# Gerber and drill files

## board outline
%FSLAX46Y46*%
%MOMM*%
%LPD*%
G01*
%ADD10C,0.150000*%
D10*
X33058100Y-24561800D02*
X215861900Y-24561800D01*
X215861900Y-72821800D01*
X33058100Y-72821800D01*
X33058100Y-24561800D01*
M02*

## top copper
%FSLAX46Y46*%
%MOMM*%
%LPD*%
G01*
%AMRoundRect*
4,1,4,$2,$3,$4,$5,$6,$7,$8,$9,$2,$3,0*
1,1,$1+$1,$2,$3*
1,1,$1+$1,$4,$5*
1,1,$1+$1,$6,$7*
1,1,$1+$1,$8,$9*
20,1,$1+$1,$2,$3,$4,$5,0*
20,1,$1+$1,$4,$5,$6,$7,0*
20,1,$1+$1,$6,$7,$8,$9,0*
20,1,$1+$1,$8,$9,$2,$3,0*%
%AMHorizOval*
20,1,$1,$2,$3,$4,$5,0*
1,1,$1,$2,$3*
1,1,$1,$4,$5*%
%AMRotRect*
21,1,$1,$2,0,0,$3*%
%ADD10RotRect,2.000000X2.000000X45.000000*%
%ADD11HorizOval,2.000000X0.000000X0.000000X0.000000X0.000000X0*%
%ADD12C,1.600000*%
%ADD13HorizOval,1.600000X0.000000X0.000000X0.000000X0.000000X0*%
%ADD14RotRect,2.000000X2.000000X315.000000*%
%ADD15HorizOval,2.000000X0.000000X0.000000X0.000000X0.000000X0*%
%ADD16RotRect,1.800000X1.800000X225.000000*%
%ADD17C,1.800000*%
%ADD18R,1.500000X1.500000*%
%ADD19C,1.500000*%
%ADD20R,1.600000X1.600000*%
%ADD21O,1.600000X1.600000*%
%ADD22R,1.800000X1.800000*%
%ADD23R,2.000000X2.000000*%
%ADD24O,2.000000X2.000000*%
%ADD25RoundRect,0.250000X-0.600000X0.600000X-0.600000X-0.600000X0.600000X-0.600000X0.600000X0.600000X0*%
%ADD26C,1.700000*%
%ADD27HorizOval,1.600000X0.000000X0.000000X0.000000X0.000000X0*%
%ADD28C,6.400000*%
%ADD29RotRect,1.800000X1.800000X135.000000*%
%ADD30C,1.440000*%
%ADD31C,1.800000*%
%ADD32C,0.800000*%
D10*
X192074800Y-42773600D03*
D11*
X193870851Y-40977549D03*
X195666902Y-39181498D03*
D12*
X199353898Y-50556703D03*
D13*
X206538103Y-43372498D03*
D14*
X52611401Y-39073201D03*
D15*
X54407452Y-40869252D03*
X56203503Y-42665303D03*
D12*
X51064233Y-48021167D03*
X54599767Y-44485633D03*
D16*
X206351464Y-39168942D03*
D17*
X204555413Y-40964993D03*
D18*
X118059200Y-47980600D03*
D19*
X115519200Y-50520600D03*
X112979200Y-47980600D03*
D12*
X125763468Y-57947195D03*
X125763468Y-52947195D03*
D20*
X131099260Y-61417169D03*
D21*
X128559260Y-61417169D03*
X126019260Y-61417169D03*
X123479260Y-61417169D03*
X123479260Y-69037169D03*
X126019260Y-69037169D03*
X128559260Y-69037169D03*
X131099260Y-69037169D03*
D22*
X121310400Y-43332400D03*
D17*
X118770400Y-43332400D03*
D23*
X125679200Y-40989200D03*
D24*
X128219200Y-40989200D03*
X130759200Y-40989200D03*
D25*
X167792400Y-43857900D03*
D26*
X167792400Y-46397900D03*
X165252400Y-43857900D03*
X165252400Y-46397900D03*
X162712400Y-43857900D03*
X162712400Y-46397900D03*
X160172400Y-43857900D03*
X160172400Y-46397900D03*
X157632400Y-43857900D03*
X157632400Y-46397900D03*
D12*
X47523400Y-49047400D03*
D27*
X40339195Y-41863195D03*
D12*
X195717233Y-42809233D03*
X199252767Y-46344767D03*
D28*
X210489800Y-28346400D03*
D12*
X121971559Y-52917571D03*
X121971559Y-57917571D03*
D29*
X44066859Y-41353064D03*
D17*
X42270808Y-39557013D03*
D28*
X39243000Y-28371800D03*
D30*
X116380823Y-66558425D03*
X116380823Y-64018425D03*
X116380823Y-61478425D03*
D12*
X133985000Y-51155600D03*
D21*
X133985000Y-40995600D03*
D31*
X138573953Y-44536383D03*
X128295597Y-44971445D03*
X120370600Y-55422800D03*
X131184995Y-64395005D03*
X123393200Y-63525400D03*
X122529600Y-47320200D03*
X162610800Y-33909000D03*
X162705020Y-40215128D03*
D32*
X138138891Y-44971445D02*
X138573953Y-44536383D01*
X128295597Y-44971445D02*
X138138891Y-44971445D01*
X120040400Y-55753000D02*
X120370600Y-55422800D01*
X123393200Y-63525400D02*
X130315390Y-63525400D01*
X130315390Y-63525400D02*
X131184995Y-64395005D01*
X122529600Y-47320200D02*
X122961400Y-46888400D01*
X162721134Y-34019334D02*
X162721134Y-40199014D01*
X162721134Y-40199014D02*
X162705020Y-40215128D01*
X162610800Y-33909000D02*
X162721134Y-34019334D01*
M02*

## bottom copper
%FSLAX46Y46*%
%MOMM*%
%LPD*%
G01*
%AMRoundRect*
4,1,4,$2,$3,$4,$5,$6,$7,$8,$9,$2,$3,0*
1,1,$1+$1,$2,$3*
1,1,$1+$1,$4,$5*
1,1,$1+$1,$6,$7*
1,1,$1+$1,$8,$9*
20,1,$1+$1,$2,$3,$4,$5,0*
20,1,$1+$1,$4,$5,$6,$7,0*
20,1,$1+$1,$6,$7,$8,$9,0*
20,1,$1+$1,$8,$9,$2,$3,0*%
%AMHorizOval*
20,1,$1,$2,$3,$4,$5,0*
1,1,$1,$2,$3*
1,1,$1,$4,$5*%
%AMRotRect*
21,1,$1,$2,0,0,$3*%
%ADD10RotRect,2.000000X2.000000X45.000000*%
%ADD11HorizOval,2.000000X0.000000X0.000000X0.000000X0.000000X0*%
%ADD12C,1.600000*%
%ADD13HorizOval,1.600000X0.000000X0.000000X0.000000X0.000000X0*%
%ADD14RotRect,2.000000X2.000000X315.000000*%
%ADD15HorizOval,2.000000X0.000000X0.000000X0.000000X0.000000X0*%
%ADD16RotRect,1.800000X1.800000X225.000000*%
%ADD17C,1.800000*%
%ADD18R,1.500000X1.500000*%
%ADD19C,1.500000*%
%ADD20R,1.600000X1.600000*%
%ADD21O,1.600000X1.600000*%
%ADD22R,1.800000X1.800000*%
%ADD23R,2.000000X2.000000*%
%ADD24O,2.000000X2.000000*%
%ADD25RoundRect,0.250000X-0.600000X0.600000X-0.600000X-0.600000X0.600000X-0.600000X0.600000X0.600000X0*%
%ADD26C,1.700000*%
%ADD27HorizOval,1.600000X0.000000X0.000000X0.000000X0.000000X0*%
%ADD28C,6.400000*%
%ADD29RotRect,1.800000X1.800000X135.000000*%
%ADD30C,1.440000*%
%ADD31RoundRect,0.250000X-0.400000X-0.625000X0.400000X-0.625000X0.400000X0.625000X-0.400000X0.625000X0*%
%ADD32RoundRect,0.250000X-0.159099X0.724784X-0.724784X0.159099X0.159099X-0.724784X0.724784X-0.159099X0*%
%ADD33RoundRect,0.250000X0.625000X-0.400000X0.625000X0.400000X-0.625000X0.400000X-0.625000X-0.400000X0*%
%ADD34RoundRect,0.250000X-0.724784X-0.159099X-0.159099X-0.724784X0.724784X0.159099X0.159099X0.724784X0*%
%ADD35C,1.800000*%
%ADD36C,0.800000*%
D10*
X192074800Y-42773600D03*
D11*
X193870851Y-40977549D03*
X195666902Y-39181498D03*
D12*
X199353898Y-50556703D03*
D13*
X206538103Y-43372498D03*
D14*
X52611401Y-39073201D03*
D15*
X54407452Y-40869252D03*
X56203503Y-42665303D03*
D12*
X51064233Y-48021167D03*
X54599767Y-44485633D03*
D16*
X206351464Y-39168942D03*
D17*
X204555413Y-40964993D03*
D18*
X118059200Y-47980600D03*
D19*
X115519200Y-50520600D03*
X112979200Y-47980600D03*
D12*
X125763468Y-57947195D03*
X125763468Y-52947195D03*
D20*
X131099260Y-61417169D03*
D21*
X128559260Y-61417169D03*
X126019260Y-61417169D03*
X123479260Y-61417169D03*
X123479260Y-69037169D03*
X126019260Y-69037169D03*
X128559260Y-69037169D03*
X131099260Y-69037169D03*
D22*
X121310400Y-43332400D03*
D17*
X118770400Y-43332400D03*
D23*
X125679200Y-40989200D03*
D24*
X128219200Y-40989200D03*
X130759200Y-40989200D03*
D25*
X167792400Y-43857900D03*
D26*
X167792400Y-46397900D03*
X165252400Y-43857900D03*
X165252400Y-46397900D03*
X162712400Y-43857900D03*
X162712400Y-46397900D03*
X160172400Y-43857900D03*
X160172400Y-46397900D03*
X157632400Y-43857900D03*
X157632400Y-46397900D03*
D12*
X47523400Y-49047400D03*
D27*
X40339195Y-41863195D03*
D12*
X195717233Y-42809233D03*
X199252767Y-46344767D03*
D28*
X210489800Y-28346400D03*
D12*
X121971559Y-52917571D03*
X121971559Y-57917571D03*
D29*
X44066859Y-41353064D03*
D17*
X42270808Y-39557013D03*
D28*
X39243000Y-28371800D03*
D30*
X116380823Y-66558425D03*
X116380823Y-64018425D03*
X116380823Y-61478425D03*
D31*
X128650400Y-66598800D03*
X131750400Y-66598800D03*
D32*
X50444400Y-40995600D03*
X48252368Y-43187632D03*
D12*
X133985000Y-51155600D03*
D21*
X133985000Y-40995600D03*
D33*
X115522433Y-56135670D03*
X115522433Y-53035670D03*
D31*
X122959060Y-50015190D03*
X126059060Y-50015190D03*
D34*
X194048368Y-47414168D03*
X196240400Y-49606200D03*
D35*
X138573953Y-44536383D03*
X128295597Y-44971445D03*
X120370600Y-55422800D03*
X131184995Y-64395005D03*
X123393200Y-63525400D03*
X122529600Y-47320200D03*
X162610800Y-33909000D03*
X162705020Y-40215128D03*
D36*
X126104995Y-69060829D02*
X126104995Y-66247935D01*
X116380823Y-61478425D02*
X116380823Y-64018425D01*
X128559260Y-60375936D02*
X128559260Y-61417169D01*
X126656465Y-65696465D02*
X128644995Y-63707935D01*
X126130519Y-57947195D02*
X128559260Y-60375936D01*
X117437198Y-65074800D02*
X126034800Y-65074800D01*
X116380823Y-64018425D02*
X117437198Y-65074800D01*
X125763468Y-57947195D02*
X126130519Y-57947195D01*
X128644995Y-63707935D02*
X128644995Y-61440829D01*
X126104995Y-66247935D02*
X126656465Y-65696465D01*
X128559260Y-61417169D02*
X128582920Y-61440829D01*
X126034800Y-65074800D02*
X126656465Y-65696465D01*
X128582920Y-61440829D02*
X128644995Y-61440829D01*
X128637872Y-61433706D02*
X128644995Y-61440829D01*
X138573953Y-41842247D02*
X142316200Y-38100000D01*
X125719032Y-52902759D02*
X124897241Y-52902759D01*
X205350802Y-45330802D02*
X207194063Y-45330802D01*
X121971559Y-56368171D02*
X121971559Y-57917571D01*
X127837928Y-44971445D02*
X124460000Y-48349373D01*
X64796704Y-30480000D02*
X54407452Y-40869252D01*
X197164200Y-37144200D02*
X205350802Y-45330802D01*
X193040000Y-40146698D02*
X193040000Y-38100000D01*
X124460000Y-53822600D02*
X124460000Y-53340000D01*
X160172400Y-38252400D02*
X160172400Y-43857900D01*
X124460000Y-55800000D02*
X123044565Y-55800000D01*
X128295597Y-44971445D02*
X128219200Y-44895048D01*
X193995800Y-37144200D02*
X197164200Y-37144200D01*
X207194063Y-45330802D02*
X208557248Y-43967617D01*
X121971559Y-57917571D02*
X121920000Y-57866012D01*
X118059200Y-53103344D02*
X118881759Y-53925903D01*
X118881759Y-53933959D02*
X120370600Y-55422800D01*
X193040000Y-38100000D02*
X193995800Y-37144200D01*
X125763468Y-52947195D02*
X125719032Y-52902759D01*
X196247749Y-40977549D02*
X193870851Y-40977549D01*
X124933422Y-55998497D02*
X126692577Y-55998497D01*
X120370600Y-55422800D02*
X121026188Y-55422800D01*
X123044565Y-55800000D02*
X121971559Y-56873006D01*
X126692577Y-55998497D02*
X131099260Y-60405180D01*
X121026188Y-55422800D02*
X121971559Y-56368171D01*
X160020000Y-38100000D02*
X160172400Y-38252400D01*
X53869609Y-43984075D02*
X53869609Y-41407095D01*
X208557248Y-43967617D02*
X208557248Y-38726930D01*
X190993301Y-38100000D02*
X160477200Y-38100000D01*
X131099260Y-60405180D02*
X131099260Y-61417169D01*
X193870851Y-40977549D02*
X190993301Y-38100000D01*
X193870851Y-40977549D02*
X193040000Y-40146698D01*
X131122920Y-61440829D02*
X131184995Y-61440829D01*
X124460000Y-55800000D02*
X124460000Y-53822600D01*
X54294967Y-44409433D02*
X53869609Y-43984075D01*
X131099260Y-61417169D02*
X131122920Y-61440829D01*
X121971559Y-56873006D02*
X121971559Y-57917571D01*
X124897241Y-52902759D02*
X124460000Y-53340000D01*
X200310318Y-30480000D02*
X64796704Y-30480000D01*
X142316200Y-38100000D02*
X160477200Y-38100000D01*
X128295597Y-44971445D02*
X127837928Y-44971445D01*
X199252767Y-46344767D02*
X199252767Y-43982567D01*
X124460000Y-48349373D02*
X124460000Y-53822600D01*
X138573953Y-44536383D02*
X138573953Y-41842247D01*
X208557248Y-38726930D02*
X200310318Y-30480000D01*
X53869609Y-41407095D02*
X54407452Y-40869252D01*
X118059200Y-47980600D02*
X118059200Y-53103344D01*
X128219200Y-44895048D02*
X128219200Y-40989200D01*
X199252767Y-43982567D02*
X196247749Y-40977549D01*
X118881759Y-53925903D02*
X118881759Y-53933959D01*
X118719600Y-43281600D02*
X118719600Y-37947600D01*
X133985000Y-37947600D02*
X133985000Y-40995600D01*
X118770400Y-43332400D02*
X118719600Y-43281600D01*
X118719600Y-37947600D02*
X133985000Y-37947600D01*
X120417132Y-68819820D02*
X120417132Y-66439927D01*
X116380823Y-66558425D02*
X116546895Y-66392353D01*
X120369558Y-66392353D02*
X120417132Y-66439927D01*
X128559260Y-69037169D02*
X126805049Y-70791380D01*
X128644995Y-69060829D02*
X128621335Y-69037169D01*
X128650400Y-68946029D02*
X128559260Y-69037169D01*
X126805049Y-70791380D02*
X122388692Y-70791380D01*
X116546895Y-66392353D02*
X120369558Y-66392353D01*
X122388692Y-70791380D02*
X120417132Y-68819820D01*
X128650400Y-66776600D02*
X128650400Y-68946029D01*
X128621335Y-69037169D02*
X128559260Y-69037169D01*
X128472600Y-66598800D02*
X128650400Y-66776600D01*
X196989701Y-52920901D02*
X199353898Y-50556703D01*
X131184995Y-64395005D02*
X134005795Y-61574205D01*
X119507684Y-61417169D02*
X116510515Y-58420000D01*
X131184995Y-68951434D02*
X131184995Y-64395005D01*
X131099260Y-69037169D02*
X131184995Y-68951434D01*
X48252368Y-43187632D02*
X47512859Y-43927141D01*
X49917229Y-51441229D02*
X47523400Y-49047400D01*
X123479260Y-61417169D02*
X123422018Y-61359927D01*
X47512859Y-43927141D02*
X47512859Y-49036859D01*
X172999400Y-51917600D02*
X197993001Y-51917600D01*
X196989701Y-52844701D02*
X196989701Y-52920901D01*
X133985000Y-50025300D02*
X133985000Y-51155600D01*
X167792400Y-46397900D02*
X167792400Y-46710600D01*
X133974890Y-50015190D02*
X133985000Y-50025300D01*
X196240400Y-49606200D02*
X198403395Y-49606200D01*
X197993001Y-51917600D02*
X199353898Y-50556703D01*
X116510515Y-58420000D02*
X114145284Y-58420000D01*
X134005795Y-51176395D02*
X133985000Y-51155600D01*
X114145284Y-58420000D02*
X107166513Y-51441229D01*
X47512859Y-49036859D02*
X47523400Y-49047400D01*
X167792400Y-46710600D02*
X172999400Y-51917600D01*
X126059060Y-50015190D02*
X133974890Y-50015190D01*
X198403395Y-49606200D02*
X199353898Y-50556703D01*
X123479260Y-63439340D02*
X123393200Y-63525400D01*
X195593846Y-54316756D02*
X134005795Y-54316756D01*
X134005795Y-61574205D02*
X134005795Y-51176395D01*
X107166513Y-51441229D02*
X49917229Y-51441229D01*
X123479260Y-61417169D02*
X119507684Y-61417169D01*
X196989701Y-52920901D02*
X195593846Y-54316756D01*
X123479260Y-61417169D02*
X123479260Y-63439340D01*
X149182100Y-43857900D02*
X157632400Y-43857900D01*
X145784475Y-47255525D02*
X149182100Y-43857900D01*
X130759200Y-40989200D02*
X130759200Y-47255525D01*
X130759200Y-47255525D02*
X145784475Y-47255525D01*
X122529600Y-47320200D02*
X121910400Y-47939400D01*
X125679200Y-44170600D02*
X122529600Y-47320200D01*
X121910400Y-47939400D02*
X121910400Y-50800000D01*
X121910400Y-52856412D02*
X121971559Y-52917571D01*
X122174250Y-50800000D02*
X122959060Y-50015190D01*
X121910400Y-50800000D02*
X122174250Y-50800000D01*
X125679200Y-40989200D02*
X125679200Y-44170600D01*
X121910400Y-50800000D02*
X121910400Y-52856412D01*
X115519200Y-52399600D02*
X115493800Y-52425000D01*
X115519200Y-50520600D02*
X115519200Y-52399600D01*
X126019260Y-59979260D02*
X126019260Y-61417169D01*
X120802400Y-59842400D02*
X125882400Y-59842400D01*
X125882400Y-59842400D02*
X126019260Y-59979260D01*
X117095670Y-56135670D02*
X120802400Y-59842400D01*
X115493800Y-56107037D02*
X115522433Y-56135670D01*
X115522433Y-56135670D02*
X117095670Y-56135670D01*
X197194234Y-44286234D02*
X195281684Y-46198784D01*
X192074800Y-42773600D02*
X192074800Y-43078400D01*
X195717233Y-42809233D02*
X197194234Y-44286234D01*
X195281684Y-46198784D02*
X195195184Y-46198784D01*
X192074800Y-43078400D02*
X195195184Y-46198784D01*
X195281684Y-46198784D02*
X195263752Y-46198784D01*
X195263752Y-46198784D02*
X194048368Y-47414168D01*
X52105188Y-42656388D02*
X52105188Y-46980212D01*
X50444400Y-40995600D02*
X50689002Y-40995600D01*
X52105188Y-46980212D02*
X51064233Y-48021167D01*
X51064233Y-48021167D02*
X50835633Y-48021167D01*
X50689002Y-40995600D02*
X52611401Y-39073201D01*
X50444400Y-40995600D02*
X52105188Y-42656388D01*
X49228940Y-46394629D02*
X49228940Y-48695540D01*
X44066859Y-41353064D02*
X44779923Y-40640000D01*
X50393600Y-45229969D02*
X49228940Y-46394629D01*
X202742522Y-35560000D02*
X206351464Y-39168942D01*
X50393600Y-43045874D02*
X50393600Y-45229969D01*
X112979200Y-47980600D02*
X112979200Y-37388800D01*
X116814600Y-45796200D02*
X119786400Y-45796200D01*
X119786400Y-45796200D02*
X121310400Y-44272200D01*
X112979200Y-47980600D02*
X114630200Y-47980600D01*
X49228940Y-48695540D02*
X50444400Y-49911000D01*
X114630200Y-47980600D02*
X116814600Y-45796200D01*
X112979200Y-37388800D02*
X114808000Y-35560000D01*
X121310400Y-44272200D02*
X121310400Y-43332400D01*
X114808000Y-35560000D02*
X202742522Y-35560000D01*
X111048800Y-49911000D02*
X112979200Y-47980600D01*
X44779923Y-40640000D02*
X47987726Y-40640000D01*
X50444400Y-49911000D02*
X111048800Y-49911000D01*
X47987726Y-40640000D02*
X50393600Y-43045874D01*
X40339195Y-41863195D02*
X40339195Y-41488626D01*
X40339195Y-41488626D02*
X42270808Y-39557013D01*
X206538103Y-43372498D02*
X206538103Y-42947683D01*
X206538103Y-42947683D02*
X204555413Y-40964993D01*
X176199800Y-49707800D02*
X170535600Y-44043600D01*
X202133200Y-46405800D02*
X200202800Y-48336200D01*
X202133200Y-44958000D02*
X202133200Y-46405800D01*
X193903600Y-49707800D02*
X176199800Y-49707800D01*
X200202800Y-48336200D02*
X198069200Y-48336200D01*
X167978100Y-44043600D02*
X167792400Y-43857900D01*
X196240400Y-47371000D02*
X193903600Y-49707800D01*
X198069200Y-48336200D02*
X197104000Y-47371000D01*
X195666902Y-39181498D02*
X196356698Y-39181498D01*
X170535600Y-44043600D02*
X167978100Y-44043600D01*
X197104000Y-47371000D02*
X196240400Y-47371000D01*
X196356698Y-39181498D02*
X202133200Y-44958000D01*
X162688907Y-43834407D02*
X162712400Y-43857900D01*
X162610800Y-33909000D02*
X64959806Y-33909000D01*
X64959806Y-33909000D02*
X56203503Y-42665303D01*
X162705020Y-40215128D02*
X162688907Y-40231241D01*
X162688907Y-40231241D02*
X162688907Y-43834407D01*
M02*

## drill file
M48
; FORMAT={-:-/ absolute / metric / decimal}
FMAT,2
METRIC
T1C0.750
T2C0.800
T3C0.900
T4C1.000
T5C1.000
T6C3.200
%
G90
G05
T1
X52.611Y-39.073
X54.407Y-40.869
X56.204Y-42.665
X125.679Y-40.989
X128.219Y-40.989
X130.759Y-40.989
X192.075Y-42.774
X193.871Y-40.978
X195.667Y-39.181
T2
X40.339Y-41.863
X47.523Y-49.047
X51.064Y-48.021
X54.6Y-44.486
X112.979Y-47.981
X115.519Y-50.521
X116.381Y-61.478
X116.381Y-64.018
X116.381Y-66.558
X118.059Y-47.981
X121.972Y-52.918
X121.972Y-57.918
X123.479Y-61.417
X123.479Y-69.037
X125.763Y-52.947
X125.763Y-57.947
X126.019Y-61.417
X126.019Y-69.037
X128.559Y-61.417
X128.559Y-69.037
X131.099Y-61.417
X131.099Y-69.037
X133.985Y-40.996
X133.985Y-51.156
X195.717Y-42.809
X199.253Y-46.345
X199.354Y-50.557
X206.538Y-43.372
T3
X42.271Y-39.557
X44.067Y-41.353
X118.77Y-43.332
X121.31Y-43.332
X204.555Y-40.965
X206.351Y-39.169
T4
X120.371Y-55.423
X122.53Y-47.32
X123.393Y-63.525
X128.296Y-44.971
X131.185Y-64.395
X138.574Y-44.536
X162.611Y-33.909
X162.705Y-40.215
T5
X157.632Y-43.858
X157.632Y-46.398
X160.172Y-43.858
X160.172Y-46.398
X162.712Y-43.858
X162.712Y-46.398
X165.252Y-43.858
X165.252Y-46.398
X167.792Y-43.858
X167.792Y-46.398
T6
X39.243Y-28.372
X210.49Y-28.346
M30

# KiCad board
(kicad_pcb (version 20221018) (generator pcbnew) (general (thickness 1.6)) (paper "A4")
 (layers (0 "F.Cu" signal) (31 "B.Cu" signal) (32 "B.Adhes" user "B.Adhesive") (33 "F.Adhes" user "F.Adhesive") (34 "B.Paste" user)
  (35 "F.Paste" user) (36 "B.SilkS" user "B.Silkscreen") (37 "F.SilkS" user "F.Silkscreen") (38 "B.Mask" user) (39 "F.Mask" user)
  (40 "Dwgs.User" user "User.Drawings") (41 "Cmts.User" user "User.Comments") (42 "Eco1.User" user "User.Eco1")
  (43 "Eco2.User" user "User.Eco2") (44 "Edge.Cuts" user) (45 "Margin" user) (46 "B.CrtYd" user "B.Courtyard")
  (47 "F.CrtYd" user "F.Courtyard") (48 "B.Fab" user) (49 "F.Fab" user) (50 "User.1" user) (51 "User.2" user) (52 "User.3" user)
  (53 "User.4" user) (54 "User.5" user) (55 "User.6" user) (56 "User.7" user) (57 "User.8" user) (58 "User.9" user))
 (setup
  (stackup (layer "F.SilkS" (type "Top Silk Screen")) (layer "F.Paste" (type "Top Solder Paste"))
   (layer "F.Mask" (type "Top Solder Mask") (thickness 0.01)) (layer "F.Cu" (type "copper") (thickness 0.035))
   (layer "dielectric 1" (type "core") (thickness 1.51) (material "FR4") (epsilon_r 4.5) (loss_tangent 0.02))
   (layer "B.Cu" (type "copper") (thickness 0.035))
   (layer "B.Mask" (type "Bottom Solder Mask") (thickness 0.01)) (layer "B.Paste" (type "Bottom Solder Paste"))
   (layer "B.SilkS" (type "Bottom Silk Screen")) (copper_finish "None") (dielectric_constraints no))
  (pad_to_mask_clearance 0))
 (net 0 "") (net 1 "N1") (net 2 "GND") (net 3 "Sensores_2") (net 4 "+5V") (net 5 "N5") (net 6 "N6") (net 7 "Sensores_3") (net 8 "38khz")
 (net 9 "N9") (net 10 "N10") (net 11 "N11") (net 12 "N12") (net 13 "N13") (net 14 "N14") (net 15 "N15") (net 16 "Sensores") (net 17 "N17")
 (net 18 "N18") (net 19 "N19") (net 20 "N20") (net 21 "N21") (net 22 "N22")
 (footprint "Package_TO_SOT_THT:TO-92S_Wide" (layer "F.Cu") (at 192.0748 42.7736 45)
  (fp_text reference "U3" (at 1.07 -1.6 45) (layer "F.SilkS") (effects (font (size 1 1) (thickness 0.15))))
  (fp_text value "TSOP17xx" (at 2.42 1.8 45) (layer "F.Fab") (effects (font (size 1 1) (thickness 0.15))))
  (pad "1" thru_hole rect (at 0 0 45) (size 2 2) (drill 0.75) (layers "*.Cu" "*.Mask") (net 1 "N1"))
  (pad "2" thru_hole oval (at 2.54 0 45) (size 2 2) (drill 0.75) (layers "*.Cu" "*.Mask") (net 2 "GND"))
  (pad "3" thru_hole oval (at 5.079999 0 45) (size 2 2) (drill 0.75) (layers "*.Cu" "*.Mask") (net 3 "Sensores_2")))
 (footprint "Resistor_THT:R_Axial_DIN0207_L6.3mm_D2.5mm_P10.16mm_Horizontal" (layer "F.Cu") (at 199.353898 50.556703 45)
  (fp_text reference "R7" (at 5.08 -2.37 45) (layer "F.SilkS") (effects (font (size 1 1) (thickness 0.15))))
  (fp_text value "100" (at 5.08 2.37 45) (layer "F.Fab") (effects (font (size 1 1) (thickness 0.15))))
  (pad "1" thru_hole circle (at 0 0 45) (size 1.6 1.6) (drill 0.8) (layers "*.Cu" "*.Mask") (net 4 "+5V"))
  (pad "2" thru_hole oval (at 10.16 0 45) (size 1.6 1.6) (drill 0.8) (layers "*.Cu" "*.Mask") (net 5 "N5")))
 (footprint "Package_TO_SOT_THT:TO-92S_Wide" (layer "F.Cu") (at 52.611401 39.073201 -45)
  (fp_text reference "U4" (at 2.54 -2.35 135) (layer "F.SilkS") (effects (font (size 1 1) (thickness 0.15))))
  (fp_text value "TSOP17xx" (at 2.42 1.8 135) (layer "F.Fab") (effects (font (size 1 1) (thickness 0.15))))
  (pad "1" thru_hole rect (at 0 0 315) (size 2 2) (drill 0.75) (layers "*.Cu" "*.Mask") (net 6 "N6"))
  (pad "2" thru_hole oval (at 2.54 0 315) (size 2 2) (drill 0.75) (layers "*.Cu" "*.Mask") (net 2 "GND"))
  (pad "3" thru_hole oval (at 5.079999 0 315) (size 2 2) (drill 0.75) (layers "*.Cu" "*.Mask") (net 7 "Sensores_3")))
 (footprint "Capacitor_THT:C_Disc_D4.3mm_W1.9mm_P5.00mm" (layer "F.Cu") (at 51.064233 48.021167 45)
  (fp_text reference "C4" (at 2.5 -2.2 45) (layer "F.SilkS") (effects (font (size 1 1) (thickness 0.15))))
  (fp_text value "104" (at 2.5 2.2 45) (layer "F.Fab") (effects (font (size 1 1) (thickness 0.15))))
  (pad "1" thru_hole circle (at 0 0 45) (size 1.6 1.6) (drill 0.8) (layers "*.Cu" "*.Mask") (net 6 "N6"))
  (pad "2" thru_hole circle (at 5 0 45) (size 1.6 1.6) (drill 0.8) (layers "*.Cu" "*.Mask") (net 2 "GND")))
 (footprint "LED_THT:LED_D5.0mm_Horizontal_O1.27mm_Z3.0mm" (layer "F.Cu") (at 206.351464 39.168942 -135)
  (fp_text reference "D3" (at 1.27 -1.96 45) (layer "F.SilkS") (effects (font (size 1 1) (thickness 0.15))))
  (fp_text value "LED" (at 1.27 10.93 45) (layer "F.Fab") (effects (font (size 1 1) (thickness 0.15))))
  (pad "1" thru_hole rect (at 0 0 225) (size 1.8 1.8) (drill 0.9) (layers "*.Cu" "*.Mask") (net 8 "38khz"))
  (pad "2" thru_hole circle (at 2.54 0 225) (size 1.8 1.8) (drill 0.9) (layers "*.Cu" "*.Mask") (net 5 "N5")))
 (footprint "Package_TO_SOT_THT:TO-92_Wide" (layer "F.Cu") (at 118.0592 47.9806 180)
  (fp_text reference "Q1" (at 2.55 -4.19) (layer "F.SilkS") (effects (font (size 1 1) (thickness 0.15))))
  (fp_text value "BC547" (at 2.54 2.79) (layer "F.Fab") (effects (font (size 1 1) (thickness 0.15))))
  (pad "1" thru_hole rect (at 0 0 180) (size 1.5 1.5) (drill 0.8) (layers "*.Cu" "*.Mask") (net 2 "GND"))
  (pad "2" thru_hole circle (at 2.54 -2.54 180) (size 1.5 1.5) (drill 0.8) (layers "*.Cu" "*.Mask") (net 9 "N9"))
  (pad "3" thru_hole circle (at 5.08 0 180) (size 1.5 1.5) (drill 0.8) (layers "*.Cu" "*.Mask") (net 8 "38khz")))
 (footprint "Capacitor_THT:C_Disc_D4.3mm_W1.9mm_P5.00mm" (layer "F.Cu") (at 125.763468 57.947195 90)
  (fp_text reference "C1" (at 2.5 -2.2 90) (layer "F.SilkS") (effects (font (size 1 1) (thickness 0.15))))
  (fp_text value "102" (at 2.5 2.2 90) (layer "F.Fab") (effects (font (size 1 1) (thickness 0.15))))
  (pad "1" thru_hole circle (at 0 0 90) (size 1.6 1.6) (drill 0.8) (layers "*.Cu" "*.Mask") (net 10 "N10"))
  (pad "2" thru_hole circle (at 5 0 90) (size 1.6 1.6) (drill 0.8) (layers "*.Cu" "*.Mask") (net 2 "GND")))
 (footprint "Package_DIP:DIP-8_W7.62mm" (layer "F.Cu") (at 131.09926 61.417169 -90)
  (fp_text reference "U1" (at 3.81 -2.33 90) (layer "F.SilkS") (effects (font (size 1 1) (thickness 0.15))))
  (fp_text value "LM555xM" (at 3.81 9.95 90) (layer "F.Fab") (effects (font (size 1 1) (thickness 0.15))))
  (pad "1" thru_hole rect (at 0 0 270) (size 1.6 1.6) (drill 0.8) (layers "*.Cu" "*.Mask") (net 2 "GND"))
  (pad "2" thru_hole oval (at 0 2.54 270) (size 1.6 1.6) (drill 0.8) (layers "*.Cu" "*.Mask") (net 10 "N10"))
  (pad "3" thru_hole oval (at 0 5.08 270) (size 1.6 1.6) (drill 0.8) (layers "*.Cu" "*.Mask") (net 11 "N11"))
  (pad "4" thru_hole oval (at 0 7.62 270) (size 1.6 1.6) (drill 0.8) (layers "*.Cu" "*.Mask") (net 4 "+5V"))
  (pad "5" thru_hole oval (at 7.62 7.62 270) (size 1.6 1.6) (drill 0.8) (layers "*.Cu" "*.Mask") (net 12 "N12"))
  (pad "6" thru_hole oval (at 7.62 5.08 270) (size 1.6 1.6) (drill 0.8) (layers "*.Cu" "*.Mask") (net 10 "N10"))
  (pad "7" thru_hole oval (at 7.62 2.54 270) (size 1.6 1.6) (drill 0.8) (layers "*.Cu" "*.Mask") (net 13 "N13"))
  (pad "8" thru_hole oval (at 7.62 0 270) (size 1.6 1.6) (drill 0.8) (layers "*.Cu" "*.Mask") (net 4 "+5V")))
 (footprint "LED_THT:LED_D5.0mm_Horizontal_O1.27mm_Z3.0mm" (layer "F.Cu") (at 121.3104 43.3324 180)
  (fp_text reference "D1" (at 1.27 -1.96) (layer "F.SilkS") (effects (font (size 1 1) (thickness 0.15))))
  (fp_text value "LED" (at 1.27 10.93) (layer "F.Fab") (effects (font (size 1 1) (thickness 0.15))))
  (pad "1" thru_hole rect (at 0 0 180) (size 1.8 1.8) (drill 0.9) (layers "*.Cu" "*.Mask") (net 8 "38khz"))
  (pad "2" thru_hole circle (at 2.54 0 180) (size 1.8 1.8) (drill 0.9) (layers "*.Cu" "*.Mask") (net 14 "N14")))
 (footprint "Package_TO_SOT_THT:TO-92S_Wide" (layer "F.Cu") (at 125.6792 40.9892)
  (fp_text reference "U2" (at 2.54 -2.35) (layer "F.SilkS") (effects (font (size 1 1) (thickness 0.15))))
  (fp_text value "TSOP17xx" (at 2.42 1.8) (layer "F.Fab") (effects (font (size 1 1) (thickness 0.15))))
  (pad "1" thru_hole rect (at 0 0) (size 2 2) (drill 0.75) (layers "*.Cu" "*.Mask") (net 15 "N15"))
  (pad "2" thru_hole oval (at 2.54 0) (size 2 2) (drill 0.75) (layers "*.Cu" "*.Mask") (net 2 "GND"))
  (pad "3" thru_hole oval (at 5.08 0) (size 2 2) (drill 0.75) (layers "*.Cu" "*.Mask") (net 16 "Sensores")))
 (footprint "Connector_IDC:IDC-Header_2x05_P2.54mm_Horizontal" (layer "F.Cu") (at 167.7924 43.8579 -90)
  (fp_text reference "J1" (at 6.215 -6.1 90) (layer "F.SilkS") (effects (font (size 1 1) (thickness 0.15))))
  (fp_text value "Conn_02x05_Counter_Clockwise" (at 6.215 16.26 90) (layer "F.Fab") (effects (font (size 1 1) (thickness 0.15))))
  (pad "1" thru_hole roundrect (at 0 0 270) (size 1.7 1.7) (drill 1) (layers "*.Cu" "*.Mask") (roundrect_rratio 0.147059)
   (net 3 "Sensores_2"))
  (pad "2" thru_hole circle (at 2.54 0 270) (size 1.7 1.7) (drill 1) (layers "*.Cu" "*.Mask") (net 4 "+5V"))
  (pad "3" thru_hole circle (at 0 2.54 270) (size 1.7 1.7) (drill 1) (layers "*.Cu" "*.Mask") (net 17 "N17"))
  (pad "4" thru_hole circle (at 2.54 2.54 270) (size 1.7 1.7) (drill 1) (layers "*.Cu" "*.Mask") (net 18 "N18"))
  (pad "5" thru_hole circle (at 0 5.08 270) (size 1.7 1.7) (drill 1) (layers "*.Cu" "*.Mask") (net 7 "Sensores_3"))
  (pad "6" thru_hole circle (at 2.54 5.08 270) (size 1.7 1.7) (drill 1) (layers "*.Cu" "*.Mask") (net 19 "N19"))
  (pad "7" thru_hole circle (at 0 7.62 270) (size 1.7 1.7) (drill 1) (layers "*.Cu" "*.Mask") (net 2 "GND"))
  (pad "8" thru_hole circle (at 2.54 7.62 270) (size 1.7 1.7) (drill 1) (layers "*.Cu" "*.Mask") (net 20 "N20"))
  (pad "9" thru_hole circle (at 0 10.16 270) (size 1.7 1.7) (drill 1) (layers "*.Cu" "*.Mask") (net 16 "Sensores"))
  (pad "10" thru_hole circle (at 2.54 10.16 270) (size 1.7 1.7) (drill 1) (layers "*.Cu" "*.Mask") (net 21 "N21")))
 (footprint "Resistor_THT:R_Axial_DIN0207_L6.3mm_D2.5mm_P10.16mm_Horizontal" (layer "F.Cu") (at 47.5234 49.0474 135)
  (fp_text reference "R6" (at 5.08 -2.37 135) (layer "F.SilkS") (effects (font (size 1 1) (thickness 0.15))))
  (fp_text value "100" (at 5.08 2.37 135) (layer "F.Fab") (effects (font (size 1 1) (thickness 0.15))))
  (pad "1" thru_hole circle (at 0 0 135) (size 1.6 1.6) (drill 0.8) (layers "*.Cu" "*.Mask") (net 4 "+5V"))
  (pad "2" thru_hole oval (at 10.16 0 135) (size 1.6 1.6) (drill 0.8) (layers "*.Cu" "*.Mask") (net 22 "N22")))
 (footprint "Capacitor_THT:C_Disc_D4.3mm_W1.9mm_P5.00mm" (layer "F.Cu") (at 195.717233 42.809233 -45)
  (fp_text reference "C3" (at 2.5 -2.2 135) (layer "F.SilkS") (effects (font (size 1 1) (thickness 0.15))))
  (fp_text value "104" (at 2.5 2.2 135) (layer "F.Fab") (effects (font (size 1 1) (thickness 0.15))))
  (pad "1" thru_hole circle (at 0 0 315) (size 1.6 1.6) (drill 0.8) (layers "*.Cu" "*.Mask") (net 1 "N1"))
  (pad "2" thru_hole circle (at 5 0 315) (size 1.6 1.6) (drill 0.8) (layers "*.Cu" "*.Mask") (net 2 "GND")))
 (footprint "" (layer "F.Cu") (at 210.4898 28.3464 180)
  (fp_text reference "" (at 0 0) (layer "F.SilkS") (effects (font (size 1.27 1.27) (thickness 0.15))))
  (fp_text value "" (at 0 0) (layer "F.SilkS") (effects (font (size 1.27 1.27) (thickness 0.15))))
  (pad "1" thru_hole circle (at 0 0 180) (size 6.4 6.4) (drill 3.2) (layers "*.Cu" "*.Mask")))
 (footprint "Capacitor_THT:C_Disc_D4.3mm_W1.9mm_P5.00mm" (layer "F.Cu") (at 121.971559 52.917571 -90)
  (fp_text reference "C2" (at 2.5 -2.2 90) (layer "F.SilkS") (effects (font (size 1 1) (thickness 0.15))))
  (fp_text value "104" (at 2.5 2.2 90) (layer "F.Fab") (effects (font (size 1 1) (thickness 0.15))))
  (pad "1" thru_hole circle (at 0 0 270) (size 1.6 1.6) (drill 0.8) (layers "*.Cu" "*.Mask") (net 15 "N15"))
  (pad "2" thru_hole circle (at 5 0 270) (size 1.6 1.6) (drill 0.8) (layers "*.Cu" "*.Mask") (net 2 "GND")))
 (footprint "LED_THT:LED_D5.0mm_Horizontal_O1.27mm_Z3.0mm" (layer "F.Cu") (at 44.066859 41.353064 135)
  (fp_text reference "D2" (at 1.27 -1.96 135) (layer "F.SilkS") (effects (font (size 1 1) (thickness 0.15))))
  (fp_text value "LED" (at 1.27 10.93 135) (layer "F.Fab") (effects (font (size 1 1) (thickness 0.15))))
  (pad "1" thru_hole rect (at 0 0 135) (size 1.8 1.8) (drill 0.9) (layers "*.Cu" "*.Mask") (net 8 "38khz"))
  (pad "2" thru_hole circle (at 2.54 0 135) (size 1.8 1.8) (drill 0.9) (layers "*.Cu" "*.Mask") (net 22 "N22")))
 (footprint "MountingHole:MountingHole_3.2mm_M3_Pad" (layer "F.Cu") (at 39.243 28.3718 180)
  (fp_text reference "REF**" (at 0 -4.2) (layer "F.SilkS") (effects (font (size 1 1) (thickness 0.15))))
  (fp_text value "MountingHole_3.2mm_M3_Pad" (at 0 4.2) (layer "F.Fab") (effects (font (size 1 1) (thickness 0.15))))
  (pad "1" thru_hole circle (at 0 0 180) (size 6.4 6.4) (drill 3.2) (layers "*.Cu" "*.Mask")))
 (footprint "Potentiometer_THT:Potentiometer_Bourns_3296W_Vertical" (layer "F.Cu") (at 116.380823 66.558425 -90)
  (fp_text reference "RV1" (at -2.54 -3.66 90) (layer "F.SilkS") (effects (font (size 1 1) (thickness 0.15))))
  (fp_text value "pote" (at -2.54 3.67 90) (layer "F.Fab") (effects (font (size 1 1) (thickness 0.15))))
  (pad "1" thru_hole circle (at 0 0 270) (size 1.44 1.44) (drill 0.8) (layers "*.Cu" "*.Mask") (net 13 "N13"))
  (pad "2" thru_hole circle (at -2.54 0 270) (size 1.44 1.44) (drill 0.8) (layers "*.Cu" "*.Mask") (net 10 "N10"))
  (pad "3" thru_hole circle (at -5.08 0 270) (size 1.44 1.44) (drill 0.8) (layers "*.Cu" "*.Mask") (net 10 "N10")))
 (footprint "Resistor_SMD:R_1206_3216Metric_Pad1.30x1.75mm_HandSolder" (layer "B.Cu") (at 130.2004 66.5988)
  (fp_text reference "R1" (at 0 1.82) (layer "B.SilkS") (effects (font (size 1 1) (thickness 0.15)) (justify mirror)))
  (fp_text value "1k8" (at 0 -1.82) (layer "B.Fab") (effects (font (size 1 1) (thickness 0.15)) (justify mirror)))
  (pad "1" smd roundrect (at -1.55 0) (size 1.3 1.75) (layers "B.Cu" "B.Paste" "B.Mask") (roundrect_rratio 0.192308) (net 13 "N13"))
  (pad "2" smd roundrect (at 1.55 0) (size 1.3 1.75) (layers "B.Cu" "B.Paste" "B.Mask") (roundrect_rratio 0.192308) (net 4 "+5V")))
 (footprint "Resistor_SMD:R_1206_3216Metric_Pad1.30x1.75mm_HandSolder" (layer "B.Cu") (at 49.348384 42.091616 -135)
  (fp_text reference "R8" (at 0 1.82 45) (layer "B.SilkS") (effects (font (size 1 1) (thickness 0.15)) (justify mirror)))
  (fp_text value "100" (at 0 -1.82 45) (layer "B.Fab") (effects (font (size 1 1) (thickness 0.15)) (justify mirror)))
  (pad "1" smd roundrect (at -1.55 0 225) (size 1.3 1.75) (layers "B.Cu" "B.Paste" "B.Mask") (roundrect_rratio 0.192308) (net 6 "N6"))
  (pad "2" smd roundrect (at 1.55 0 225) (size 1.3 1.75) (layers "B.Cu" "B.Paste" "B.Mask") (roundrect_rratio 0.192308) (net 4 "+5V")))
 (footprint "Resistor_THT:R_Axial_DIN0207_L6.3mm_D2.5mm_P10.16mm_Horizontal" (layer "B.Cu") (at 133.985 51.1556 90)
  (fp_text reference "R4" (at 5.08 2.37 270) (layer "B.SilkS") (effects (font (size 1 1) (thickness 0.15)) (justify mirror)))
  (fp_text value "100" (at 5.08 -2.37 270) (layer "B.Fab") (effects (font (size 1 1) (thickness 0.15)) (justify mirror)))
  (pad "1" thru_hole circle (at 0 0 90) (size 1.6 1.6) (drill 0.8) (layers "*.Cu" "*.Mask") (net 4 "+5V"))
  (pad "2" thru_hole oval (at 10.16 0 90) (size 1.6 1.6) (drill 0.8) (layers "*.Cu" "*.Mask") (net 14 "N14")))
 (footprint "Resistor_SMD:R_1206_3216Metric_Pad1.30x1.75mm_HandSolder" (layer "B.Cu") (at 115.522433 54.58567 90)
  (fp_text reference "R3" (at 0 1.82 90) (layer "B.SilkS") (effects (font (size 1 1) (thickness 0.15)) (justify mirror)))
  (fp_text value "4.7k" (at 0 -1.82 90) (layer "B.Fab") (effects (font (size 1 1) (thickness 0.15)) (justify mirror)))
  (pad "1" smd roundrect (at -1.55 0 90) (size 1.3 1.75) (layers "B.Cu" "B.Paste" "B.Mask") (roundrect_rratio 0.192308) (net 11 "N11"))
  (pad "2" smd roundrect (at 1.55 0 90) (size 1.3 1.75) (layers "B.Cu" "B.Paste" "B.Mask") (roundrect_rratio 0.192308) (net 9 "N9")))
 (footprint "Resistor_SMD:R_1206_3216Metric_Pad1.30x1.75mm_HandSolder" (layer "B.Cu") (at 124.50906 50.01519)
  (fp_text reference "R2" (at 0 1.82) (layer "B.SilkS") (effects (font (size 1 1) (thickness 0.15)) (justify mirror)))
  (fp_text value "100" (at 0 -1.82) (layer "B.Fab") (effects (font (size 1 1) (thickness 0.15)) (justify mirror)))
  (pad "1" smd roundrect (at -1.55 0) (size 1.3 1.75) (layers "B.Cu" "B.Paste" "B.Mask") (roundrect_rratio 0.192308) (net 15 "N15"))
  (pad "2" smd roundrect (at 1.55 0) (size 1.3 1.75) (layers "B.Cu" "B.Paste" "B.Mask") (roundrect_rratio 0.192308) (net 4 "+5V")))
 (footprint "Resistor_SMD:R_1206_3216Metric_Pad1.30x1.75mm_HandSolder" (layer "B.Cu") (at 195.144384 48.510184 -45)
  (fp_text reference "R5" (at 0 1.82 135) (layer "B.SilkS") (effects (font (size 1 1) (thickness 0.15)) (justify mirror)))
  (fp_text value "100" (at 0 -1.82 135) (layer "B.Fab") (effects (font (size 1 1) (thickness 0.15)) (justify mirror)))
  (pad "1" smd roundrect (at -1.55 0 315) (size 1.3 1.75) (layers "B.Cu" "B.Paste" "B.Mask") (roundrect_rratio 0.192308) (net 1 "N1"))
  (pad "2" smd roundrect (at 1.55 0 315) (size 1.3 1.75) (layers "B.Cu" "B.Paste" "B.Mask") (roundrect_rratio 0.192308) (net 4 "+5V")))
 (gr_rect (start 33.0581 24.5618) (end 215.8619 72.8218) (stroke (width 0.15) (type default)) (fill none) (layer "Edge.Cuts"))
 (segment (start 126.104995 69.060829) (end 126.104995 66.247935) (width 0.8) (layer "B.Cu") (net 10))
 (segment (start 116.380823 61.478425) (end 116.380823 64.018425) (width 0.8) (layer "B.Cu") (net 10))
 (segment (start 128.55926 60.375936) (end 128.55926 61.417169) (width 0.8) (layer "B.Cu") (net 10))
 (segment (start 126.656465 65.696465) (end 128.644995 63.707935) (width 0.8) (layer "B.Cu") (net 10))
 (segment (start 126.130519 57.947195) (end 128.55926 60.375936) (width 0.8) (layer "B.Cu") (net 10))
 (segment (start 117.437198 65.0748) (end 126.0348 65.0748) (width 0.8) (layer "B.Cu") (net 10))
 (segment (start 116.380823 64.018425) (end 117.437198 65.0748) (width 0.8) (layer "B.Cu") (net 10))
 (segment (start 125.763468 57.947195) (end 126.130519 57.947195) (width 0.8) (layer "B.Cu") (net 10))
 (segment (start 128.644995 63.707935) (end 128.644995 61.440829) (width 0.8) (layer "B.Cu") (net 10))
 (segment (start 126.104995 66.247935) (end 126.656465 65.696465) (width 0.8) (layer "B.Cu") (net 10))
 (segment (start 128.55926 61.417169) (end 128.58292 61.440829) (width 0.8) (layer "B.Cu") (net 10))
 (segment (start 126.0348 65.0748) (end 126.656465 65.696465) (width 0.8) (layer "B.Cu") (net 10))
 (segment (start 128.58292 61.440829) (end 128.644995 61.440829) (width 0.8) (layer "B.Cu") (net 10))
 (segment (start 128.637872 61.433706) (end 128.644995 61.440829) (width 0.8) (layer "B.Cu") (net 10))
 (segment (start 138.138891 44.971445) (end 138.573953 44.536383) (width 0.8) (layer "F.Cu") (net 2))
 (segment (start 128.295597 44.971445) (end 138.138891 44.971445) (width 0.8) (layer "F.Cu") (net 2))
 (segment (start 120.0404 55.753) (end 120.3706 55.4228) (width 0.8) (layer "F.Cu") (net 2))
 (via (at 138.573953 44.536383) (size 1.8) (drill 1) (layers "F.Cu" "B.Cu") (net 2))
 (via (at 128.295597 44.971445) (size 1.8) (drill 1) (layers "F.Cu" "B.Cu") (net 2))
 (via (at 120.3706 55.4228) (size 1.8) (drill 1) (layers "F.Cu" "B.Cu") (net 2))
 (segment (start 138.573953 41.842247) (end 142.3162 38.1) (width 0.8) (layer "B.Cu") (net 2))
 (segment (start 125.719032 52.902759) (end 124.897241 52.902759) (width 0.8) (layer "B.Cu") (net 2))
 (segment (start 205.350802 45.330802) (end 207.194063 45.330802) (width 0.8) (layer "B.Cu") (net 2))
 (segment (start 121.971559 56.368171) (end 121.971559 57.917571) (width 0.8) (layer "B.Cu") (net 2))
 (segment (start 127.837928 44.971445) (end 124.46 48.349373) (width 0.8) (layer "B.Cu") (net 2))
 (segment (start 64.796704 30.48) (end 54.407452 40.869252) (width 0.8) (layer "B.Cu") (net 2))
 (segment (start 197.1642 37.1442) (end 205.350802 45.330802) (width 0.8) (layer "B.Cu") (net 2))
 (segment (start 193.04 40.146698) (end 193.04 38.1) (width 0.8) (layer "B.Cu") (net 2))
 (segment (start 124.46 53.8226) (end 124.46 53.34) (width 0.8) (layer "B.Cu") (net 2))
 (segment (start 160.1724 38.2524) (end 160.1724 43.8579) (width 0.8) (layer "B.Cu") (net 2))
 (segment (start 124.46 55.8) (end 123.044565 55.8) (width 0.8) (layer "B.Cu") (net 2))
 (segment (start 128.295597 44.971445) (end 128.2192 44.895048) (width 0.8) (layer "B.Cu") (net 2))
 (segment (start 193.9958 37.1442) (end 197.1642 37.1442) (width 0.8) (layer "B.Cu") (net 2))
 (segment (start 207.194063 45.330802) (end 208.557248 43.967617) (width 0.8) (layer "B.Cu") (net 2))
 (segment (start 121.971559 57.917571) (end 121.92 57.866012) (width 0.8) (layer "B.Cu") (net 2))
 (segment (start 118.0592 53.103344) (end 118.881759 53.925903) (width 0.8) (layer "B.Cu") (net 2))
 (segment (start 118.881759 53.933959) (end 120.3706 55.4228) (width 0.8) (layer "B.Cu") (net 2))
 (segment (start 193.04 38.1) (end 193.9958 37.1442) (width 0.8) (layer "B.Cu") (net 2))
 (segment (start 125.763468 52.947195) (end 125.719032 52.902759) (width 0.8) (layer "B.Cu") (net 2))
 (segment (start 196.247749 40.977549) (end 193.870851 40.977549) (width 0.8) (layer "B.Cu") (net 2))
 (segment (start 124.933422 55.998497) (end 126.692577 55.998497) (width 0.8) (layer "B.Cu") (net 2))
 (segment (start 120.3706 55.4228) (end 121.026188 55.4228) (width 0.8) (layer "B.Cu") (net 2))
 (segment (start 123.044565 55.8) (end 121.971559 56.873006) (width 0.8) (layer "B.Cu") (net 2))
 (segment (start 126.692577 55.998497) (end 131.09926 60.40518) (width 0.8) (layer "B.Cu") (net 2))
 (segment (start 121.026188 55.4228) (end 121.971559 56.368171) (width 0.8) (layer "B.Cu") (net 2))
 (segment (start 160.02 38.1) (end 160.1724 38.2524) (width 0.8) (layer "B.Cu") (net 2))
 (segment (start 53.869609 43.984075) (end 53.869609 41.407095) (width 0.8) (layer "B.Cu") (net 2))
 (segment (start 208.557248 43.967617) (end 208.557248 38.72693) (width 0.8) (layer "B.Cu") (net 2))
 (segment (start 190.993301 38.1) (end 160.4772 38.1) (width 0.8) (layer "B.Cu") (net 2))
 (segment (start 131.09926 60.40518) (end 131.09926 61.417169) (width 0.8) (layer "B.Cu") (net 2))
 (segment (start 193.870851 40.977549) (end 190.993301 38.1) (width 0.8) (layer "B.Cu") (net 2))
 (segment (start 193.870851 40.977549) (end 193.04 40.146698) (width 0.8) (layer "B.Cu") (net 2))
 (segment (start 131.12292 61.440829) (end 131.184995 61.440829) (width 0.8) (layer "B.Cu") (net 2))
 (segment (start 124.46 55.8) (end 124.46 53.8226) (width 0.8) (layer "B.Cu") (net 2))
 (segment (start 54.294967 44.409433) (end 53.869609 43.984075) (width 0.8) (layer "B.Cu") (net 2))
 (segment (start 131.09926 61.417169) (end 131.12292 61.440829) (width 0.8) (layer "B.Cu") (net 2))
 (segment (start 121.971559 56.873006) (end 121.971559 57.917571) (width 0.8) (layer "B.Cu") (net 2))
 (segment (start 124.897241 52.902759) (end 124.46 53.34) (width 0.8) (layer "B.Cu") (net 2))
 (segment (start 200.310318 30.48) (end 64.796704 30.48) (width 0.8) (layer "B.Cu") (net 2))
 (segment (start 142.3162 38.1) (end 160.4772 38.1) (width 0.8) (layer "B.Cu") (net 2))
 (segment (start 128.295597 44.971445) (end 127.837928 44.971445) (width 0.8) (layer "B.Cu") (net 2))
 (segment (start 199.252767 46.344767) (end 199.252767 43.982567) (width 0.8) (layer "B.Cu") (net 2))
 (segment (start 124.46 48.349373) (end 124.46 53.8226) (width 0.8) (layer "B.Cu") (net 2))
 (segment (start 138.573953 44.536383) (end 138.573953 41.842247) (width 0.8) (layer "B.Cu") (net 2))
 (segment (start 208.557248 38.72693) (end 200.310318 30.48) (width 0.8) (layer "B.Cu") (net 2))
 (segment (start 53.869609 41.407095) (end 54.407452 40.869252) (width 0.8) (layer "B.Cu") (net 2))
 (segment (start 118.0592 47.9806) (end 118.0592 53.103344) (width 0.8) (layer "B.Cu") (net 2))
 (segment (start 128.2192 44.895048) (end 128.2192 40.9892) (width 0.8) (layer "B.Cu") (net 2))
 (segment (start 199.252767 43.982567) (end 196.247749 40.977549) (width 0.8) (layer "B.Cu") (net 2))
 (segment (start 118.881759 53.925903) (end 118.881759 53.933959) (width 0.8) (layer "B.Cu") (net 2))
 (segment (start 118.7196 43.2816) (end 118.7196 37.9476) (width 0.8) (layer "B.Cu") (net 14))
 (segment (start 133.985 37.9476) (end 133.985 40.9956) (width 0.8) (layer "B.Cu") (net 14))
 (segment (start 118.7704 43.3324) (end 118.7196 43.2816) (width 0.8) (layer "B.Cu") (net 14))
 (segment (start 118.7196 37.9476) (end 133.985 37.9476) (width 0.8) (layer "B.Cu") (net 14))
 (segment (start 120.417132 68.81982) (end 120.417132 66.439927) (width 0.8) (layer "B.Cu") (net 13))
 (segment (start 116.380823 66.558425) (end 116.546895 66.392353) (width 0.8) (layer "B.Cu") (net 13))
 (segment (start 120.369558 66.392353) (end 120.417132 66.439927) (width 0.8) (layer "B.Cu") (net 13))
 (segment (start 128.55926 69.037169) (end 126.805049 70.79138) (width 0.8) (layer "B.Cu") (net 13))
 (segment (start 128.644995 69.060829) (end 128.621335 69.037169) (width 0.8) (layer "B.Cu") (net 13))
 (segment (start 128.6504 68.946029) (end 128.55926 69.037169) (width 0.8) (layer "B.Cu") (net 13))
 (segment (start 126.805049 70.79138) (end 122.388692 70.79138) (width 0.8) (layer "B.Cu") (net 13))
 (segment (start 116.546895 66.392353) (end 120.369558 66.392353) (width 0.8) (layer "B.Cu") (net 13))
 (segment (start 122.388692 70.79138) (end 120.417132 68.81982) (width 0.8) (layer "B.Cu") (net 13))
 (segment (start 128.6504 66.7766) (end 128.6504 68.946029) (width 0.8) (layer "B.Cu") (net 13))
 (segment (start 128.621335 69.037169) (end 128.55926 69.037169) (width 0.8) (layer "B.Cu") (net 13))
 (segment (start 128.4726 66.5988) (end 128.6504 66.7766) (width 0.8) (layer "B.Cu") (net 13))
 (segment (start 123.3932 63.5254) (end 130.31539 63.5254) (width 0.8) (layer "F.Cu") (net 4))
 (segment (start 130.31539 63.5254) (end 131.184995 64.395005) (width 0.8) (layer "F.Cu") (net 4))
 (via (at 131.184995 64.395005) (size 1.8) (drill 1) (layers "F.Cu" "B.Cu") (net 4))
 (via (at 123.3932 63.5254) (size 1.8) (drill 1) (layers "F.Cu" "B.Cu") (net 4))
 (segment (start 196.989701 52.920901) (end 199.353898 50.556703) (width 0.8) (layer "B.Cu") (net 4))
 (segment (start 131.184995 64.395005) (end 134.005795 61.574205) (width 0.8) (layer "B.Cu") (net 4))
 (segment (start 119.507684 61.417169) (end 116.510515 58.42) (width 0.8) (layer "B.Cu") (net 4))
 (segment (start 131.184995 68.951434) (end 131.184995 64.395005) (width 0.8) (layer "B.Cu") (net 4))
 (segment (start 131.09926 69.037169) (end 131.184995 68.951434) (width 0.8) (layer "B.Cu") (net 4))
 (segment (start 48.252368 43.187632) (end 47.512859 43.927141) (width 0.8) (layer "B.Cu") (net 4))
 (segment (start 49.917229 51.441229) (end 47.5234 49.0474) (width 0.8) (layer "B.Cu") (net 4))
 (segment (start 123.47926 61.417169) (end 123.422018 61.359927) (width 0.8) (layer "B.Cu") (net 4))
 (segment (start 47.512859 43.927141) (end 47.512859 49.036859) (width 0.8) (layer "B.Cu") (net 4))
 (segment (start 172.9994 51.9176) (end 197.993001 51.9176) (width 0.8) (layer "B.Cu") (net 4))
 (segment (start 196.989701 52.844701) (end 196.989701 52.920901) (width 0.8) (layer "B.Cu") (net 4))
 (segment (start 133.985 50.0253) (end 133.985 51.1556) (width 0.8) (layer "B.Cu") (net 4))
 (segment (start 167.7924 46.3979) (end 167.7924 46.7106) (width 0.8) (layer "B.Cu") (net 4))
 (segment (start 133.97489 50.01519) (end 133.985 50.0253) (width 0.8) (layer "B.Cu") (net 4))
 (segment (start 196.2404 49.6062) (end 198.403395 49.6062) (width 0.8) (layer "B.Cu") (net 4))
 (segment (start 197.993001 51.9176) (end 199.353898 50.556703) (width 0.8) (layer "B.Cu") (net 4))
 (segment (start 116.510515 58.42) (end 114.145284 58.42) (width 0.8) (layer "B.Cu") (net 4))
 (segment (start 134.005795 51.176395) (end 133.985 51.1556) (width 0.8) (layer "B.Cu") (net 4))
 (segment (start 114.145284 58.42) (end 107.166513 51.441229) (width 0.8) (layer "B.Cu") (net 4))
 (segment (start 47.512859 49.036859) (end 47.5234 49.0474) (width 0.8) (layer "B.Cu") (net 4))
 (segment (start 167.7924 46.7106) (end 172.9994 51.9176) (width 0.8) (layer "B.Cu") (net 4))
 (segment (start 126.05906 50.01519) (end 133.97489 50.01519) (width 0.8) (layer "B.Cu") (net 4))
 (segment (start 198.403395 49.6062) (end 199.353898 50.556703) (width 0.8) (layer "B.Cu") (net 4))
 (segment (start 123.47926 63.43934) (end 123.3932 63.5254) (width 0.8) (layer "B.Cu") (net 4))
 (segment (start 195.593846 54.316756) (end 134.005795 54.316756) (width 0.8) (layer "B.Cu") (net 4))
 (segment (start 134.005795 61.574205) (end 134.005795 51.176395) (width 0.8) (layer "B.Cu") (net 4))
 (segment (start 107.166513 51.441229) (end 49.917229 51.441229) (width 0.8) (layer "B.Cu") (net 4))
 (segment (start 123.47926 61.417169) (end 119.507684 61.417169) (width 0.8) (layer "B.Cu") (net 4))
 (segment (start 196.989701 52.920901) (end 195.593846 54.316756) (width 0.8) (layer "B.Cu") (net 4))
 (segment (start 123.47926 61.417169) (end 123.47926 63.43934) (width 0.8) (layer "B.Cu") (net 4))
 (segment (start 149.1821 43.8579) (end 157.6324 43.8579) (width 0.8) (layer "B.Cu") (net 16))
 (segment (start 145.784475 47.255525) (end 149.1821 43.8579) (width 0.8) (layer "B.Cu") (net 16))
 (segment (start 130.7592 40.9892) (end 130.7592 47.255525) (width 0.8) (layer "B.Cu") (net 16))
 (segment (start 130.7592 47.255525) (end 145.784475 47.255525) (width 0.8) (layer "B.Cu") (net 16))
 (segment (start 122.5296 47.3202) (end 122.9614 46.8884) (width 0.8) (layer "F.Cu") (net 15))
 (via (at 122.5296 47.3202) (size 1.8) (drill 1) (layers "F.Cu" "B.Cu") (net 15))
 (segment (start 122.5296 47.3202) (end 121.9104 47.9394) (width 0.8) (layer "B.Cu") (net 15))
 (segment (start 125.6792 44.1706) (end 122.5296 47.3202) (width 0.8) (layer "B.Cu") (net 15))
 (segment (start 121.9104 47.9394) (end 121.9104 50.8) (width 0.8) (layer "B.Cu") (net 15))
 (segment (start 121.9104 52.856412) (end 121.971559 52.917571) (width 0.8) (layer "B.Cu") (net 15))
 (segment (start 122.17425 50.8) (end 122.95906 50.01519) (width 0.8) (layer "B.Cu") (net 15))
 (segment (start 121.9104 50.8) (end 122.17425 50.8) (width 0.8) (layer "B.Cu") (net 15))
 (segment (start 125.6792 40.9892) (end 125.6792 44.1706) (width 0.8) (layer "B.Cu") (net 15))
 (segment (start 121.9104 50.8) (end 121.9104 52.856412) (width 0.8) (layer "B.Cu") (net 15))
 (segment (start 115.5192 52.3996) (end 115.4938 52.425) (width 0.8) (layer "B.Cu") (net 9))
 (segment (start 115.5192 50.5206) (end 115.5192 52.3996) (width 0.8) (layer "B.Cu") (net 9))
 (segment (start 126.01926 59.97926) (end 126.01926 61.417169) (width 0.8) (layer "B.Cu") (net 11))
 (segment (start 120.8024 59.8424) (end 125.8824 59.8424) (width 0.8) (layer "B.Cu") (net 11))
 (segment (start 125.8824 59.8424) (end 126.01926 59.97926) (width 0.8) (layer "B.Cu") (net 11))
 (segment (start 117.09567 56.13567) (end 120.8024 59.8424) (width 0.8) (layer "B.Cu") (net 11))
 (segment (start 115.4938 56.107037) (end 115.522433 56.13567) (width 0.8) (layer "B.Cu") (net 11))
 (segment (start 115.522433 56.13567) (end 117.09567 56.13567) (width 0.8) (layer "B.Cu") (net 11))
 (segment (start 197.194234 44.286234) (end 195.281684 46.198784) (width 0.8) (layer "B.Cu") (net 1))
 (segment (start 192.0748 42.7736) (end 192.0748 43.0784) (width 0.8) (layer "B.Cu") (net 1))
 (segment (start 195.717233 42.809233) (end 197.194234 44.286234) (width 0.8) (layer "B.Cu") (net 1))
 (segment (start 195.281684 46.198784) (end 195.195184 46.198784) (width 0.8) (layer "B.Cu") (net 1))
 (segment (start 192.0748 43.0784) (end 195.195184 46.198784) (width 0.8) (layer "B.Cu") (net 1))
 (segment (start 195.281684 46.198784) (end 195.263752 46.198784) (width 0.8) (layer "B.Cu") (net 1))
 (segment (start 195.263752 46.198784) (end 194.048368 47.414168) (width 0.8) (layer "B.Cu") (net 1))
 (segment (start 52.105188 42.656388) (end 52.105188 46.980212) (width 0.8) (layer "B.Cu") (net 6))
 (segment (start 50.4444 40.9956) (end 50.689002 40.9956) (width 0.8) (layer "B.Cu") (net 6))
 (segment (start 52.105188 46.980212) (end 51.064233 48.021167) (width 0.8) (layer "B.Cu") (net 6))
 (segment (start 51.064233 48.021167) (end 50.835633 48.021167) (width 0.8) (layer "B.Cu") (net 6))
 (segment (start 50.689002 40.9956) (end 52.611401 39.073201) (width 0.8) (layer "B.Cu") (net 6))
 (segment (start 50.4444 40.9956) (end 52.105188 42.656388) (width 0.8) (layer "B.Cu") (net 6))
 (segment (start 49.22894 46.394629) (end 49.22894 48.69554) (width 0.8) (layer "B.Cu") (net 8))
 (segment (start 44.066859 41.353064) (end 44.779923 40.64) (width 0.8) (layer "B.Cu") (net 8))
 (segment (start 50.3936 45.229969) (end 49.22894 46.394629) (width 0.8) (layer "B.Cu") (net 8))
 (segment (start 202.742522 35.56) (end 206.351464 39.168942) (width 0.8) (layer "B.Cu") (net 8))
 (segment (start 50.3936 43.045874) (end 50.3936 45.229969) (width 0.8) (layer "B.Cu") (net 8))
 (segment (start 112.9792 47.9806) (end 112.9792 37.3888) (width 0.8) (layer "B.Cu") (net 8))
 (segment (start 116.8146 45.7962) (end 119.7864 45.7962) (width 0.8) (layer "B.Cu") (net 8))
 (segment (start 119.7864 45.7962) (end 121.3104 44.2722) (width 0.8) (layer "B.Cu") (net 8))
 (segment (start 112.9792 47.9806) (end 114.6302 47.9806) (width 0.8) (layer "B.Cu") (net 8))
 (segment (start 49.22894 48.69554) (end 50.4444 49.911) (width 0.8) (layer "B.Cu") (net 8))
 (segment (start 114.6302 47.9806) (end 116.8146 45.7962) (width 0.8) (layer "B.Cu") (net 8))
 (segment (start 112.9792 37.3888) (end 114.808 35.56) (width 0.8) (layer "B.Cu") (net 8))
 (segment (start 121.3104 44.2722) (end 121.3104 43.3324) (width 0.8) (layer "B.Cu") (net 8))
 (segment (start 114.808 35.56) (end 202.742522 35.56) (width 0.8) (layer "B.Cu") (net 8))
 (segment (start 111.0488 49.911) (end 112.9792 47.9806) (width 0.8) (layer "B.Cu") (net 8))
 (segment (start 44.779923 40.64) (end 47.987726 40.64) (width 0.8) (layer "B.Cu") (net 8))
 (segment (start 50.4444 49.911) (end 111.0488 49.911) (width 0.8) (layer "B.Cu") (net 8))
 (segment (start 47.987726 40.64) (end 50.3936 43.045874) (width 0.8) (layer "B.Cu") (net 8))
 (segment (start 40.339195 41.863195) (end 40.339195 41.488626) (width 0.8) (layer "B.Cu") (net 22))
 (segment (start 40.339195 41.488626) (end 42.270808 39.557013) (width 0.8) (layer "B.Cu") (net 22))
 (segment (start 206.538103 43.372498) (end 206.538103 42.947683) (width 0.8) (layer "B.Cu") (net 5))
 (segment (start 206.538103 42.947683) (end 204.555413 40.964993) (width 0.8) (layer "B.Cu") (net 5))
 (segment (start 176.1998 49.7078) (end 170.5356 44.0436) (width 0.8) (layer "B.Cu") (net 3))
 (segment (start 202.1332 46.4058) (end 200.2028 48.3362) (width 0.8) (layer "B.Cu") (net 3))
 (segment (start 202.1332 44.958) (end 202.1332 46.4058) (width 0.8) (layer "B.Cu") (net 3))
 (segment (start 193.9036 49.7078) (end 176.1998 49.7078) (width 0.8) (layer "B.Cu") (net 3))
 (segment (start 200.2028 48.3362) (end 198.0692 48.3362) (width 0.8) (layer "B.Cu") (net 3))
 (segment (start 167.9781 44.0436) (end 167.7924 43.8579) (width 0.8) (layer "B.Cu") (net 3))
 (segment (start 196.2404 47.371) (end 193.9036 49.7078) (width 0.8) (layer "B.Cu") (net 3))
 (segment (start 198.0692 48.3362) (end 197.104 47.371) (width 0.8) (layer "B.Cu") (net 3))
 (segment (start 195.666902 39.181498) (end 196.356698 39.181498) (width 0.8) (layer "B.Cu") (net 3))
 (segment (start 170.5356 44.0436) (end 167.9781 44.0436) (width 0.8) (layer "B.Cu") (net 3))
 (segment (start 197.104 47.371) (end 196.2404 47.371) (width 0.8) (layer "B.Cu") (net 3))
 (segment (start 196.356698 39.181498) (end 202.1332 44.958) (width 0.8) (layer "B.Cu") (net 3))
 (segment (start 162.721134 34.019334) (end 162.721134 40.199014) (width 0.8) (layer "F.Cu") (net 7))
 (segment (start 162.721134 40.199014) (end 162.70502 40.215128) (width 0.8) (layer "F.Cu") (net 7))
 (segment (start 162.6108 33.909) (end 162.721134 34.019334) (width 0.8) (layer "F.Cu") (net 7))
 (via (at 162.6108 33.909) (size 1.8) (drill 1) (layers "F.Cu" "B.Cu") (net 7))
 (via (at 162.70502 40.215128) (size 1.8) (drill 1) (layers "F.Cu" "B.Cu") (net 7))
 (segment (start 162.688907 43.834407) (end 162.7124 43.8579) (width 0.8) (layer "B.Cu") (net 7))
 (segment (start 162.6108 33.909) (end 64.959806 33.909) (width 0.8) (layer "B.Cu") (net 7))
 (segment (start 64.959806 33.909) (end 56.203503 42.665303) (width 0.8) (layer "B.Cu") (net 7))
 (segment (start 162.70502 40.215128) (end 162.688907 40.231241) (width 0.8) (layer "B.Cu") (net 7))
 (segment (start 162.688907 40.231241) (end 162.688907 43.834407) (width 0.8) (layer "B.Cu") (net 7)))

